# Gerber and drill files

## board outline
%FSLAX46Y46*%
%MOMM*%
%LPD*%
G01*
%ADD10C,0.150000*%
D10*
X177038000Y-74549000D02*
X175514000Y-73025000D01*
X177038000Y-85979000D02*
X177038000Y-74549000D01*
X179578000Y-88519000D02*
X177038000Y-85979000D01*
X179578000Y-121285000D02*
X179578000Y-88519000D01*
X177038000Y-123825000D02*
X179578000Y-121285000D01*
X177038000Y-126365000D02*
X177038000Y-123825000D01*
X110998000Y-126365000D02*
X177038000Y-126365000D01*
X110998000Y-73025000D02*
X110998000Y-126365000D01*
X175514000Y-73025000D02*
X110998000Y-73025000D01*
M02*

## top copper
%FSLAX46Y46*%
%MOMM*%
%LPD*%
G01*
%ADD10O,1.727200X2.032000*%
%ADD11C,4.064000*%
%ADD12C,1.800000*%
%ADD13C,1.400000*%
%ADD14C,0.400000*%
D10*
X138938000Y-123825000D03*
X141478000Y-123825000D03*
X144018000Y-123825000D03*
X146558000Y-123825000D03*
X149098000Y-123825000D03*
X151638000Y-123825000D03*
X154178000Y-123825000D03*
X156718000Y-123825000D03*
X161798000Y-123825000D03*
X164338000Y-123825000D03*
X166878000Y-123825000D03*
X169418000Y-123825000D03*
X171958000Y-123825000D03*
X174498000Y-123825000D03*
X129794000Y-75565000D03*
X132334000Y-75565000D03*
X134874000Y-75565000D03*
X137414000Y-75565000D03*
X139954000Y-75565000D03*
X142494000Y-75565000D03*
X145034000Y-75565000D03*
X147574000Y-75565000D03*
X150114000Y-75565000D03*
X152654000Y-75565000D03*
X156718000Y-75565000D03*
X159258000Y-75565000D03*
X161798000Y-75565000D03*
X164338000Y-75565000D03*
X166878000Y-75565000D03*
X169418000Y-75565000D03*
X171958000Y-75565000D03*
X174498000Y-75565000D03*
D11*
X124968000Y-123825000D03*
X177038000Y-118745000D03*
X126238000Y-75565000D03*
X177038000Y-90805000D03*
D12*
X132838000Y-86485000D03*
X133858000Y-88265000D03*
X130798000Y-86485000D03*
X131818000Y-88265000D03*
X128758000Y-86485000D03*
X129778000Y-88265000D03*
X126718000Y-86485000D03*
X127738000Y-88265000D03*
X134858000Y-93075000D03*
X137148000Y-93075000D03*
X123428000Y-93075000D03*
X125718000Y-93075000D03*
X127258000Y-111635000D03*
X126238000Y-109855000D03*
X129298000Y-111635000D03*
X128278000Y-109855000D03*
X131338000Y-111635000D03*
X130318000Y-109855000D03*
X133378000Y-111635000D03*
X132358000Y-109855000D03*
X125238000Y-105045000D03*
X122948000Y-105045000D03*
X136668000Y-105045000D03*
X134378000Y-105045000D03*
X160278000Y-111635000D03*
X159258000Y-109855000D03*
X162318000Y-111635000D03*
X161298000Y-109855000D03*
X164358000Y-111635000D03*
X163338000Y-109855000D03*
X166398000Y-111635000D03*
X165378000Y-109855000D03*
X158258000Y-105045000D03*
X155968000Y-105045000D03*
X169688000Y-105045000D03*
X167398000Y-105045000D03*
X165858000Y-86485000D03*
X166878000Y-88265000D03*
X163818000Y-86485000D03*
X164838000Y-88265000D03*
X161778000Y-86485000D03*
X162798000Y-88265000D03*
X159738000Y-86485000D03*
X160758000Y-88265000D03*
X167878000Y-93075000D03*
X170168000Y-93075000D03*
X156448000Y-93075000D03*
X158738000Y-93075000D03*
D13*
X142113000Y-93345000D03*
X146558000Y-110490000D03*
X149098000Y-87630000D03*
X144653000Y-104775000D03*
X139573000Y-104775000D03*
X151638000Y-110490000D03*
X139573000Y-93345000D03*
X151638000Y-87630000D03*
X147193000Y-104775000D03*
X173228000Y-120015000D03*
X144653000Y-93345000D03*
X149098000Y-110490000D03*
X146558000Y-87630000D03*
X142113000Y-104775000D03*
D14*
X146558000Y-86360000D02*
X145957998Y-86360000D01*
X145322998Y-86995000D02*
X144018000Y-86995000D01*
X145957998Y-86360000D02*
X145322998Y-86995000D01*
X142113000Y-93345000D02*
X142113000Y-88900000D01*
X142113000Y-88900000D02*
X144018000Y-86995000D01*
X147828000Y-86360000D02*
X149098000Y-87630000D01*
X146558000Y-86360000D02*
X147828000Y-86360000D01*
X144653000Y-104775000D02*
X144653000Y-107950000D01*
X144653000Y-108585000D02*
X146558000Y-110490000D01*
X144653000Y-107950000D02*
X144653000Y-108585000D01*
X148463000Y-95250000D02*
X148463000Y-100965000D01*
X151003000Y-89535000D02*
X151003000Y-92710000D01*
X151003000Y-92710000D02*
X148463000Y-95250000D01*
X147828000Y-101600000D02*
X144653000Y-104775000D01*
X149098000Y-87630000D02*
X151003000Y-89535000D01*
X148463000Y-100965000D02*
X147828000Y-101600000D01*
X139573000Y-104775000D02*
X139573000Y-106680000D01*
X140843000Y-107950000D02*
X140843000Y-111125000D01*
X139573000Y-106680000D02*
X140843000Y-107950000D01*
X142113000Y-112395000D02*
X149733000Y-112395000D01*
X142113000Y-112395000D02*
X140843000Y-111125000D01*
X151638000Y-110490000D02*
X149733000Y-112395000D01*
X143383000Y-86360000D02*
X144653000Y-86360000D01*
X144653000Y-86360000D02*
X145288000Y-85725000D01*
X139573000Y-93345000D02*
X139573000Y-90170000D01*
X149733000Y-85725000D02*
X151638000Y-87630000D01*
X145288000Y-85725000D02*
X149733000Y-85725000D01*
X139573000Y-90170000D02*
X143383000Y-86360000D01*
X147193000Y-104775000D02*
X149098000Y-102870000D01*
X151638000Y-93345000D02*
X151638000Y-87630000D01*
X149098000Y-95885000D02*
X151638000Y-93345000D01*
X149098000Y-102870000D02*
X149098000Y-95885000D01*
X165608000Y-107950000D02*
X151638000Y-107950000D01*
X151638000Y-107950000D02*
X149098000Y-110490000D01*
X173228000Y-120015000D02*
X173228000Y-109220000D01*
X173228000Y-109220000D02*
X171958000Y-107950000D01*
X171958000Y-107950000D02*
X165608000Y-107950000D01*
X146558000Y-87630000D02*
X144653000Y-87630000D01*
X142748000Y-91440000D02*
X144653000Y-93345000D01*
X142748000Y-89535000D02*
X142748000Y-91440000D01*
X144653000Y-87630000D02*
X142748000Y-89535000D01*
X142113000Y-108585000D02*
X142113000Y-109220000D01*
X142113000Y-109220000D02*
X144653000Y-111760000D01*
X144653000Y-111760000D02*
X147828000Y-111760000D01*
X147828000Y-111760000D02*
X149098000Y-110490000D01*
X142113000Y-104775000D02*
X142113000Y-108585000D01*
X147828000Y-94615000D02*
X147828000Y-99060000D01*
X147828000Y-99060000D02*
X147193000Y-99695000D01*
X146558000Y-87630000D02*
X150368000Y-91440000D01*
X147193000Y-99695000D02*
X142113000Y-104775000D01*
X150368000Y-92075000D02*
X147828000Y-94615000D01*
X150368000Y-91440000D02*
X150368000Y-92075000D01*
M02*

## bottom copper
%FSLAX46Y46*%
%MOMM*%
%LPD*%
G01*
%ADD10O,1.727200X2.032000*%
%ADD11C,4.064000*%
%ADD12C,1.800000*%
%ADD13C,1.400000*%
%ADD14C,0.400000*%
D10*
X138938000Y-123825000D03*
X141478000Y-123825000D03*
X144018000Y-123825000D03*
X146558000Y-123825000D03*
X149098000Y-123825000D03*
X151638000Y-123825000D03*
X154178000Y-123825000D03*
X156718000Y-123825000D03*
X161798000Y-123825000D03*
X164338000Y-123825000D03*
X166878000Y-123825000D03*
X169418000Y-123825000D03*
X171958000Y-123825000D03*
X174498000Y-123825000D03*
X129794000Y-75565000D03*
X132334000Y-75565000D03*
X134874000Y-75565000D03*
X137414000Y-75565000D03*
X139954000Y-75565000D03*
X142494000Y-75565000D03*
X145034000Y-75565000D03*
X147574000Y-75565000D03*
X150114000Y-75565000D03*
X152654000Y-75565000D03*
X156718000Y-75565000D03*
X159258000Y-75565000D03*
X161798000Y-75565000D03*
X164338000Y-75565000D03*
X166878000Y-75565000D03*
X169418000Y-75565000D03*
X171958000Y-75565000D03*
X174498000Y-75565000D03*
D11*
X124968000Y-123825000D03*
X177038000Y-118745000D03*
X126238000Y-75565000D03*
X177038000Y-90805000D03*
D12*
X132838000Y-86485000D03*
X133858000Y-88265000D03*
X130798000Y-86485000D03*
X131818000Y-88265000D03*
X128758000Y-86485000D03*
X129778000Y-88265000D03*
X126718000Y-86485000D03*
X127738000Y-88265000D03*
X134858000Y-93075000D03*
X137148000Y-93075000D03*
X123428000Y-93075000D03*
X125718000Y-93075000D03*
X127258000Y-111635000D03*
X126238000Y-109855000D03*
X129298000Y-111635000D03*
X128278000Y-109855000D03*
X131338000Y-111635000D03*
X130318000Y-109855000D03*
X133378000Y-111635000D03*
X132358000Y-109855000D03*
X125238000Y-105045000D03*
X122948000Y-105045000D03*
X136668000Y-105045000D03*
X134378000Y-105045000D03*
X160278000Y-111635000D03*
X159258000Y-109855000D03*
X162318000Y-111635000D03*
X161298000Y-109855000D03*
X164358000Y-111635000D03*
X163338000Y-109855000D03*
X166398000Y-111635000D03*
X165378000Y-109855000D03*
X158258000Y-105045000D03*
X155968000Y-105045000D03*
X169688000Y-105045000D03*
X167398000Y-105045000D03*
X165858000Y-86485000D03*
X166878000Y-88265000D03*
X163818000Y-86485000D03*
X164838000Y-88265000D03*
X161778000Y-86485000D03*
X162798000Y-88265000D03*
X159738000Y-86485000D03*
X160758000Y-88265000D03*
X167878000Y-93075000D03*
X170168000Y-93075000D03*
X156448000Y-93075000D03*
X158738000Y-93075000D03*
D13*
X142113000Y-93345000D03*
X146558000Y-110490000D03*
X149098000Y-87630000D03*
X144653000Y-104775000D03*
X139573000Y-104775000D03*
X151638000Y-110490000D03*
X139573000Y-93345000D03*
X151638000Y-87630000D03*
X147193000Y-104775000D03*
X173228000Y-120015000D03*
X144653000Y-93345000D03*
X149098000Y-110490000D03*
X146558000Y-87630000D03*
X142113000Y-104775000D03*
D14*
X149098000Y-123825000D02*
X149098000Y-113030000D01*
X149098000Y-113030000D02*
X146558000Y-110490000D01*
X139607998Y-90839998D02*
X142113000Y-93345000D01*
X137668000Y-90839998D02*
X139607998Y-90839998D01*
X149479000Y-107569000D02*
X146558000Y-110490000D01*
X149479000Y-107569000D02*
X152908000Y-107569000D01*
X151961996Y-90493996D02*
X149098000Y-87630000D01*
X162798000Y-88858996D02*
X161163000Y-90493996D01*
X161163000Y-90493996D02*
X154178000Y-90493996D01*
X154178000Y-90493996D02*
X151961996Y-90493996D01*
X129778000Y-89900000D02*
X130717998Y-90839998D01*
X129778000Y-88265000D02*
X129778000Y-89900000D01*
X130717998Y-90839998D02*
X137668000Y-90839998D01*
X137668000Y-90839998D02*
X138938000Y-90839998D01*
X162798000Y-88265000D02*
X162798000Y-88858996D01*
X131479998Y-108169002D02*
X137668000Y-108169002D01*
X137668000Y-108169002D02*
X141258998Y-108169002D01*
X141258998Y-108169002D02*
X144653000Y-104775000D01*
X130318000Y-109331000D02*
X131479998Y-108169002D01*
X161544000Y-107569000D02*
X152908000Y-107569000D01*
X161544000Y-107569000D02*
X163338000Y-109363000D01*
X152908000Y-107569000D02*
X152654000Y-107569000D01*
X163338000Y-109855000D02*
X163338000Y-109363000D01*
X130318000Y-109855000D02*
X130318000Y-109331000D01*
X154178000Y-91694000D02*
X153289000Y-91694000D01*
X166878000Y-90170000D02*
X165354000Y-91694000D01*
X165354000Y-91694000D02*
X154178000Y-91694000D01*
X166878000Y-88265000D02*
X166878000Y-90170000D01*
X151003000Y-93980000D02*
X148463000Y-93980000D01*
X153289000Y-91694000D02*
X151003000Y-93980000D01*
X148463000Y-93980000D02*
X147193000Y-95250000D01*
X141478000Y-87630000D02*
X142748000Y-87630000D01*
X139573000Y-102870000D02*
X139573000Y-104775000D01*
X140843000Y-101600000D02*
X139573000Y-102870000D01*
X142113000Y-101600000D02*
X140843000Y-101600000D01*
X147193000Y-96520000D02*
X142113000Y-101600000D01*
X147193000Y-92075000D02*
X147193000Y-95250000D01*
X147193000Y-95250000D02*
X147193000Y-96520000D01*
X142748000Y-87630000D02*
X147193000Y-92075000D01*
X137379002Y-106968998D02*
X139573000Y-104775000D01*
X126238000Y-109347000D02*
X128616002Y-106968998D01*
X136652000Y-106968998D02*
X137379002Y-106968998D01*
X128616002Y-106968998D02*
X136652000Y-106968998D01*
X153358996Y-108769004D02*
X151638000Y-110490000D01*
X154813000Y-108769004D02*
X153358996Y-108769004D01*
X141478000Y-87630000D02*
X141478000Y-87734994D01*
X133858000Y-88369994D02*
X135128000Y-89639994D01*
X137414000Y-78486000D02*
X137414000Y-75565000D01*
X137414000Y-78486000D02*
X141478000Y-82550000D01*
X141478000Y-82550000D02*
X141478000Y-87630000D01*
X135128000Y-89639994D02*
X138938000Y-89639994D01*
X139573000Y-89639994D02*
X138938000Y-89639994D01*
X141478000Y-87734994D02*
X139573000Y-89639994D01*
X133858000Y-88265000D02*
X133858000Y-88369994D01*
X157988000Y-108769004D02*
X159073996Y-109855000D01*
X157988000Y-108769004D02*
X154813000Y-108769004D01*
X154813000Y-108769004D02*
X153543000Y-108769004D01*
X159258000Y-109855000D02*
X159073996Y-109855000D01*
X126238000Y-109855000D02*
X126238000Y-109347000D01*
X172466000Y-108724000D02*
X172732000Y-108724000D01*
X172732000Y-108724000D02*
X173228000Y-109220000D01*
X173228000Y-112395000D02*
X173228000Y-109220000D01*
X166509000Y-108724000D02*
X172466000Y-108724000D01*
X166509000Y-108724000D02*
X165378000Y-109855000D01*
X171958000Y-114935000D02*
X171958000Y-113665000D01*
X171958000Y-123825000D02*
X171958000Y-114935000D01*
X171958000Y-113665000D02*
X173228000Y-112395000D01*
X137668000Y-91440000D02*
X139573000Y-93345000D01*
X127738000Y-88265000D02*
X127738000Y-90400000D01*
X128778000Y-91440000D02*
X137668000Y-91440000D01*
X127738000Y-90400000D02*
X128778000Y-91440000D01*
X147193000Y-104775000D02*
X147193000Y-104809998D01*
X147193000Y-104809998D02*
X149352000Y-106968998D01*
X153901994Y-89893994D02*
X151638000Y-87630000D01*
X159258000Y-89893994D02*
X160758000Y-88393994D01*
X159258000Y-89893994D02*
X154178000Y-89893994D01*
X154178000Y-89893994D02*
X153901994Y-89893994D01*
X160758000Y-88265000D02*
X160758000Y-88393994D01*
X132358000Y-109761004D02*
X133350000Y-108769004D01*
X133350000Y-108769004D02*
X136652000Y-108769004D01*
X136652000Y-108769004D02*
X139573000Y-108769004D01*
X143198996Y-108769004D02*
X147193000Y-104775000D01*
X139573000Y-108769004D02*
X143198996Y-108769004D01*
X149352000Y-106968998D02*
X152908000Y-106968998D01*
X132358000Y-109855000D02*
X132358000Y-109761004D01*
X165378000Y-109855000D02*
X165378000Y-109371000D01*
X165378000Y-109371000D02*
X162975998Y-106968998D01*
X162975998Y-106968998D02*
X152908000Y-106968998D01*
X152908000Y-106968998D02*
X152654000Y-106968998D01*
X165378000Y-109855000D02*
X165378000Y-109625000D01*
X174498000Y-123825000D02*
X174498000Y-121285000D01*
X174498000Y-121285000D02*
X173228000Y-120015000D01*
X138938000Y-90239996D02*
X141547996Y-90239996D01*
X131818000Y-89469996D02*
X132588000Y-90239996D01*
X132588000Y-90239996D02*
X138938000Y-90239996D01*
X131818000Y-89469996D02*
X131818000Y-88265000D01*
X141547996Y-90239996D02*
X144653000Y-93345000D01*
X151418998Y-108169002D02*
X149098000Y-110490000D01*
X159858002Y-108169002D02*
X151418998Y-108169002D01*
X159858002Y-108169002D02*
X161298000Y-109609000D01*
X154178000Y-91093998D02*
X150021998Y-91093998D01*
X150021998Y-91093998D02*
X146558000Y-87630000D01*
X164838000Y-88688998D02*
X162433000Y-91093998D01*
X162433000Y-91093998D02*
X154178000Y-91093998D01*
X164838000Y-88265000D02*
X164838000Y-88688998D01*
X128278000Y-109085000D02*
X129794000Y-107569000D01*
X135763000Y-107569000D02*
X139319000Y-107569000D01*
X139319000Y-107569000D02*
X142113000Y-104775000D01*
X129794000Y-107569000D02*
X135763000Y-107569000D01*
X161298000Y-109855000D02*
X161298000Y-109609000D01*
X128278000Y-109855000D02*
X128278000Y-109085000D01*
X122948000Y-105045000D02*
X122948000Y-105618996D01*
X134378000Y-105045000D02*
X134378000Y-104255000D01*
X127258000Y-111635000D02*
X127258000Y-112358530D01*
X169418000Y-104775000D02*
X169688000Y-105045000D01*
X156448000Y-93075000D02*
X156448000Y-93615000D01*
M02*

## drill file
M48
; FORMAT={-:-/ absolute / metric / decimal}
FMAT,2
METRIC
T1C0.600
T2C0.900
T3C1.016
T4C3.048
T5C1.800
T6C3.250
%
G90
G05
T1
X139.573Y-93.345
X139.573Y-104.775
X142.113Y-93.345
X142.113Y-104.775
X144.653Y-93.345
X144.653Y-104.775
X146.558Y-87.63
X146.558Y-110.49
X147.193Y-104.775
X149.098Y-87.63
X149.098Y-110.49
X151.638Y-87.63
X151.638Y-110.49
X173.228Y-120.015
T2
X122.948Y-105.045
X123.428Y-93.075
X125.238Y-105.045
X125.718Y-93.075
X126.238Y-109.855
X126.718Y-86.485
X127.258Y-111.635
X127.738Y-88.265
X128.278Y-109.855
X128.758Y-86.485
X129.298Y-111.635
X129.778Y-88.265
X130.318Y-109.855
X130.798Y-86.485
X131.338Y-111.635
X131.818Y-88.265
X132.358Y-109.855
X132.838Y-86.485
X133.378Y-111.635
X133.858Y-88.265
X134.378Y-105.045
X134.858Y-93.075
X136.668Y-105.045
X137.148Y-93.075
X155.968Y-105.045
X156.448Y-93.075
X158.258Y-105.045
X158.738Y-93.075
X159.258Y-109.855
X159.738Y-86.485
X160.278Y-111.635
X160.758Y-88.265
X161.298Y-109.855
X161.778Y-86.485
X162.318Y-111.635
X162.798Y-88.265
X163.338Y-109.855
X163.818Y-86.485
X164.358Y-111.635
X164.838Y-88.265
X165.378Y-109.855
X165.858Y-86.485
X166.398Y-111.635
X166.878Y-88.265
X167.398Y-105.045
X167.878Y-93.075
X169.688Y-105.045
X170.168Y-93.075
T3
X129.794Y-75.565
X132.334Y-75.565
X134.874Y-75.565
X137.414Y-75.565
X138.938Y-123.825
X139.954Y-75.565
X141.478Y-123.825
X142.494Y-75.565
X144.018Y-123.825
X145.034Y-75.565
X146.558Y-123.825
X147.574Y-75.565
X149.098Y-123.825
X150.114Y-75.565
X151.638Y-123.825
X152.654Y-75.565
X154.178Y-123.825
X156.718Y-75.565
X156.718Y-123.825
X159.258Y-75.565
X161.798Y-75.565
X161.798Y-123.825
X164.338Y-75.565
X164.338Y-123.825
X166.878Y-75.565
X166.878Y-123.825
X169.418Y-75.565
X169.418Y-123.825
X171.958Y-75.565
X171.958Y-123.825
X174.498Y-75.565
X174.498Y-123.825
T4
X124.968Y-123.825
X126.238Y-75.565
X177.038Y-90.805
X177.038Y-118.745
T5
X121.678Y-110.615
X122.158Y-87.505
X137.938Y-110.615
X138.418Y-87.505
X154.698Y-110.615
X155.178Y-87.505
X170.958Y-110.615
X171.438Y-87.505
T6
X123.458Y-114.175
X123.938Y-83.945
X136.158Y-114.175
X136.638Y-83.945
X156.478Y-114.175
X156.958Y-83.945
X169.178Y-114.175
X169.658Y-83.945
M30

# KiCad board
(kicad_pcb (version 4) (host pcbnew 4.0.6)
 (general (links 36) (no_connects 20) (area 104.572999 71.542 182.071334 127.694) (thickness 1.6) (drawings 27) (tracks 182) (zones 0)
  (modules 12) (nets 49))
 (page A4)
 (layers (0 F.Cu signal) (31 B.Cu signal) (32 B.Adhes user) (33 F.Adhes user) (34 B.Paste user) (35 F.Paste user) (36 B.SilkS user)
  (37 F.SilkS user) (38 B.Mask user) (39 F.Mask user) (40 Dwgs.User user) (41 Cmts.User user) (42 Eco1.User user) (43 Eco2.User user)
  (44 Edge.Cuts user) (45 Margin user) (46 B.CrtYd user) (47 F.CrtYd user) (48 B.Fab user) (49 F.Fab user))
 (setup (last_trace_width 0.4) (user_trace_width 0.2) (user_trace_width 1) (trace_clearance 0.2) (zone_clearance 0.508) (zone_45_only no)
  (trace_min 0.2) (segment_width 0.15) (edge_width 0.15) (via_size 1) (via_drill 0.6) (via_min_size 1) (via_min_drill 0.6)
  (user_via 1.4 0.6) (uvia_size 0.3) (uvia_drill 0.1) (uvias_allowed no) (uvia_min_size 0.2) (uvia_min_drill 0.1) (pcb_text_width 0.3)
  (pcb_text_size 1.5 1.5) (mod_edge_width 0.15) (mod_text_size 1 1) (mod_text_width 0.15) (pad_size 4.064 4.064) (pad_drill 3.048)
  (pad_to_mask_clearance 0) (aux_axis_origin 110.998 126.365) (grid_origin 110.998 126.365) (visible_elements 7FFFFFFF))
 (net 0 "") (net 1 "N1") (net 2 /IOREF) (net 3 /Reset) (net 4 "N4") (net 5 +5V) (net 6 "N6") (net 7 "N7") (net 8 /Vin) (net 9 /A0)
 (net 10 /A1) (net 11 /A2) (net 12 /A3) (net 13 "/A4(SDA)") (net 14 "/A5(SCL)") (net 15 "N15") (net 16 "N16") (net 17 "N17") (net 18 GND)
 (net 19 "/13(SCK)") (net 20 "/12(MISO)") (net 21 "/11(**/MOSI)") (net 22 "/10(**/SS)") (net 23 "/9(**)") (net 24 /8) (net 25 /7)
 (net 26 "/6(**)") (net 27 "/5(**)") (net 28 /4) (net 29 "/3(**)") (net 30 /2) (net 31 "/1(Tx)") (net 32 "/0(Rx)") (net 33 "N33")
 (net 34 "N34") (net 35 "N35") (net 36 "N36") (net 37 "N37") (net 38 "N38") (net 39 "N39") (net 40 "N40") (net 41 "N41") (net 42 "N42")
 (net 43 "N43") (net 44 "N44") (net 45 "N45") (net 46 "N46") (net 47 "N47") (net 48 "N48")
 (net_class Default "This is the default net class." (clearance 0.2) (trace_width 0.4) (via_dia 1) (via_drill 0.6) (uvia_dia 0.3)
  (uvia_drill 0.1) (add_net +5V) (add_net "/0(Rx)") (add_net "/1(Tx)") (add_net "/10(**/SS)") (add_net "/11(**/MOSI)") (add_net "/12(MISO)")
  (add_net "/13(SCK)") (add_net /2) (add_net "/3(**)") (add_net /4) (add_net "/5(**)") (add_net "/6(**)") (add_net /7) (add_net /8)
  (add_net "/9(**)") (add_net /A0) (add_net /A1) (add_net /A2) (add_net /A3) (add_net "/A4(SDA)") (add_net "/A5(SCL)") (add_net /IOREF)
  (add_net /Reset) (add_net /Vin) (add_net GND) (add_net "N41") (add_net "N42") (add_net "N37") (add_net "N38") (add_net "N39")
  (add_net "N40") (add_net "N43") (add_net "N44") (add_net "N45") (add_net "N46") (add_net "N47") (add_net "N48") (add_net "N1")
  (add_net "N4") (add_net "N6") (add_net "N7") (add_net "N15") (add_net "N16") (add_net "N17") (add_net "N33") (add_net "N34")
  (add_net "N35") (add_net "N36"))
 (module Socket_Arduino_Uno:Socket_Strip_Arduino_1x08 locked (layer F.Cu) (at 138.938 123.825)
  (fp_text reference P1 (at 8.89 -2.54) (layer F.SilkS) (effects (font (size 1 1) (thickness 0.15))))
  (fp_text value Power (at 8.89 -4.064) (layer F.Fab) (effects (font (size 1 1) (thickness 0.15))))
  (pad 1 thru_hole oval (at 0 0) (size 1.7272 2.032) (drill 1.016) (layers *.Cu *.Mask F.SilkS) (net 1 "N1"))
  (pad 2 thru_hole oval (at 2.54 0) (size 1.7272 2.032) (drill 1.016) (layers *.Cu *.Mask F.SilkS) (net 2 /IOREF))
  (pad 3 thru_hole oval (at 5.08 0) (size 1.7272 2.032) (drill 1.016) (layers *.Cu *.Mask F.SilkS) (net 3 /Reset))
  (pad 4 thru_hole oval (at 7.62 0) (size 1.7272 2.032) (drill 1.016) (layers *.Cu *.Mask F.SilkS) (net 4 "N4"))
  (pad 5 thru_hole oval (at 10.16 0) (size 1.7272 2.032) (drill 1.016) (layers *.Cu *.Mask F.SilkS) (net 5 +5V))
  (pad 6 thru_hole oval (at 12.7 0) (size 1.7272 2.032) (drill 1.016) (layers *.Cu *.Mask F.SilkS) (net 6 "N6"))
  (pad 7 thru_hole oval (at 15.24 0) (size 1.7272 2.032) (drill 1.016) (layers *.Cu *.Mask F.SilkS) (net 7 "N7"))
  (pad 8 thru_hole oval (at 17.78 0) (size 1.7272 2.032) (drill 1.016) (layers *.Cu *.Mask F.SilkS) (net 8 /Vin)))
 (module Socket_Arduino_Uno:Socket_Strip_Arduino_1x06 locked (layer F.Cu) (at 161.798 123.825)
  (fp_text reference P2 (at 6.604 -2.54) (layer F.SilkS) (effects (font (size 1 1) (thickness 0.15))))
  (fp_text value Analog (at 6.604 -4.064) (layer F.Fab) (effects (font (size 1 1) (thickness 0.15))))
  (pad 1 thru_hole oval (at 0 0) (size 1.7272 2.032) (drill 1.016) (layers *.Cu *.Mask F.SilkS) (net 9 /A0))
  (pad 2 thru_hole oval (at 2.54 0) (size 1.7272 2.032) (drill 1.016) (layers *.Cu *.Mask F.SilkS) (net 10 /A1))
  (pad 3 thru_hole oval (at 5.08 0) (size 1.7272 2.032) (drill 1.016) (layers *.Cu *.Mask F.SilkS) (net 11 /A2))
  (pad 4 thru_hole oval (at 7.62 0) (size 1.7272 2.032) (drill 1.016) (layers *.Cu *.Mask F.SilkS) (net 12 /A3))
  (pad 5 thru_hole oval (at 10.16 0) (size 1.7272 2.032) (drill 1.016) (layers *.Cu *.Mask F.SilkS) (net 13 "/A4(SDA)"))
  (pad 6 thru_hole oval (at 12.7 0) (size 1.7272 2.032) (drill 1.016) (layers *.Cu *.Mask F.SilkS) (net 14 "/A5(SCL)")))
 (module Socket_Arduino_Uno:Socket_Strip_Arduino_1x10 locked (layer F.Cu) (at 129.794 75.565)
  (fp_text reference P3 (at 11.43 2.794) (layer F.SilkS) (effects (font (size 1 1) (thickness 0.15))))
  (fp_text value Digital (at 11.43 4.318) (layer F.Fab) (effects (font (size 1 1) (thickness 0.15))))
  (pad 1 thru_hole oval (at 0 0) (size 1.7272 2.032) (drill 1.016) (layers *.Cu *.Mask F.SilkS) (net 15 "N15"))
  (pad 2 thru_hole oval (at 2.54 0) (size 1.7272 2.032) (drill 1.016) (layers *.Cu *.Mask F.SilkS) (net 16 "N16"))
  (pad 3 thru_hole oval (at 5.08 0) (size 1.7272 2.032) (drill 1.016) (layers *.Cu *.Mask F.SilkS) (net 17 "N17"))
  (pad 4 thru_hole oval (at 7.62 0) (size 1.7272 2.032) (drill 1.016) (layers *.Cu *.Mask F.SilkS) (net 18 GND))
  (pad 5 thru_hole oval (at 10.16 0) (size 1.7272 2.032) (drill 1.016) (layers *.Cu *.Mask F.SilkS) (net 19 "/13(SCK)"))
  (pad 6 thru_hole oval (at 12.7 0) (size 1.7272 2.032) (drill 1.016) (layers *.Cu *.Mask F.SilkS) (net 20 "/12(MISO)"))
  (pad 7 thru_hole oval (at 15.24 0) (size 1.7272 2.032) (drill 1.016) (layers *.Cu *.Mask F.SilkS) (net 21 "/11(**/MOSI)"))
  (pad 8 thru_hole oval (at 17.78 0) (size 1.7272 2.032) (drill 1.016) (layers *.Cu *.Mask F.SilkS) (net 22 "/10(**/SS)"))
  (pad 9 thru_hole oval (at 20.32 0) (size 1.7272 2.032) (drill 1.016) (layers *.Cu *.Mask F.SilkS) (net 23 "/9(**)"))
  (pad 10 thru_hole oval (at 22.86 0) (size 1.7272 2.032) (drill 1.016) (layers *.Cu *.Mask F.SilkS) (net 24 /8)))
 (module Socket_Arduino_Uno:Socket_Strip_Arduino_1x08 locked (layer F.Cu) (at 156.718 75.565)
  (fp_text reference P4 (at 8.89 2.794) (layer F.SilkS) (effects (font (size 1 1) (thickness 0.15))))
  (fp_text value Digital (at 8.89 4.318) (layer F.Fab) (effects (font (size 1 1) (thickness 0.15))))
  (pad 1 thru_hole oval (at 0 0) (size 1.7272 2.032) (drill 1.016) (layers *.Cu *.Mask F.SilkS) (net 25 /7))
  (pad 2 thru_hole oval (at 2.54 0) (size 1.7272 2.032) (drill 1.016) (layers *.Cu *.Mask F.SilkS) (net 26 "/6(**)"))
  (pad 3 thru_hole oval (at 5.08 0) (size 1.7272 2.032) (drill 1.016) (layers *.Cu *.Mask F.SilkS) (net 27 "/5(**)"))
  (pad 4 thru_hole oval (at 7.62 0) (size 1.7272 2.032) (drill 1.016) (layers *.Cu *.Mask F.SilkS) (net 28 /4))
  (pad 5 thru_hole oval (at 10.16 0) (size 1.7272 2.032) (drill 1.016) (layers *.Cu *.Mask F.SilkS) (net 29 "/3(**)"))
  (pad 6 thru_hole oval (at 12.7 0) (size 1.7272 2.032) (drill 1.016) (layers *.Cu *.Mask F.SilkS) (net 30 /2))
  (pad 7 thru_hole oval (at 15.24 0) (size 1.7272 2.032) (drill 1.016) (layers *.Cu *.Mask F.SilkS) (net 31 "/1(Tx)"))
  (pad 8 thru_hole oval (at 17.78 0) (size 1.7272 2.032) (drill 1.016) (layers *.Cu *.Mask F.SilkS) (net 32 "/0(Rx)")))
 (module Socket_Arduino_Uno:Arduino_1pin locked (layer F.Cu) (at 124.968 123.825)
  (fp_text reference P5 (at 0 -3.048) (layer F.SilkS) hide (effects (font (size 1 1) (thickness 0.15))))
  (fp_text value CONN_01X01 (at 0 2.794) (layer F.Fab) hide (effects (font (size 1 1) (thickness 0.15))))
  (pad 1 thru_hole circle (at 0 0) (size 4.064 4.064) (drill 3.048) (layers *.Cu *.Mask F.SilkS) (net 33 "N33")))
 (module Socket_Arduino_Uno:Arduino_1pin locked (layer F.Cu) (at 177.038 118.745)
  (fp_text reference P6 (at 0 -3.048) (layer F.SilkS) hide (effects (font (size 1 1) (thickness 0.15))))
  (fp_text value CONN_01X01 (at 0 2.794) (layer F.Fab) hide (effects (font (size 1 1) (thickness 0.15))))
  (pad 1 thru_hole circle (at 0 0) (size 4.064 4.064) (drill 3.048) (layers *.Cu *.Mask F.SilkS) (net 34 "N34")))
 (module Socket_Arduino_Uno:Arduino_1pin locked (layer F.Cu) (at 126.238 75.565)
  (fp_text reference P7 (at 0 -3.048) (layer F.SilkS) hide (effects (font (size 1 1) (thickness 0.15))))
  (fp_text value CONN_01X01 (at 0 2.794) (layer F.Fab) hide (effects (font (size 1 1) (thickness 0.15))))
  (pad 1 thru_hole circle (at 0 0) (size 4.064 4.064) (drill 3.048) (layers *.Cu *.Mask F.SilkS) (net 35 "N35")))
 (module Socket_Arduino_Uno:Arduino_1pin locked (layer F.Cu) (at 177.038 90.805)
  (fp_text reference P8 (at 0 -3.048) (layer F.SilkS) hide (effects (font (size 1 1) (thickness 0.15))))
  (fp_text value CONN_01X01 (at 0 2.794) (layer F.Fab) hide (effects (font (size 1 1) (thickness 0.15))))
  (pad 1 thru_hole circle (at 0 0) (size 4.064 4.064) (drill 3.048) (layers *.Cu *.Mask F.SilkS) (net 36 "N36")))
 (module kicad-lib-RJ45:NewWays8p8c (layer F.Cu) (at 133.858 88.265 180)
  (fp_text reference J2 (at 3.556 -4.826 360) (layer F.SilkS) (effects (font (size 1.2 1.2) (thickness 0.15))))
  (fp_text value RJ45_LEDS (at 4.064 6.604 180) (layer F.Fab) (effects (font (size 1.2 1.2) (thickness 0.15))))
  (pad 2 thru_hole circle (at 1.02 1.78 180) (size 1.8 1.8) (drill 0.9) (layers *.Cu *.Mask) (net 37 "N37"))
  (pad 1 thru_hole circle (at 0 0 180) (size 1.8 1.8) (drill 0.9) (layers *.Cu *.Mask) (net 18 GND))
  (pad 4 thru_hole circle (at 3.06 1.78 180) (size 1.8 1.8) (drill 0.9) (layers *.Cu *.Mask) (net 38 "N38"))
  (pad 3 thru_hole circle (at 2.04 0 180) (size 1.8 1.8) (drill 0.9) (layers *.Cu *.Mask) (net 14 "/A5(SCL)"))
  (pad 6 thru_hole circle (at 5.1 1.78 180) (size 1.8 1.8) (drill 0.9) (layers *.Cu *.Mask) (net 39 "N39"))
  (pad 5 thru_hole circle (at 4.08 0 180) (size 1.8 1.8) (drill 0.9) (layers *.Cu *.Mask) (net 5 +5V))
  (pad 8 thru_hole circle (at 7.14 1.78 180) (size 1.8 1.8) (drill 0.9) (layers *.Cu *.Mask) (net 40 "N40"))
  (pad 7 thru_hole circle (at 6.12 0 180) (size 1.8 1.8) (drill 0.9) (layers *.Cu *.Mask) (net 13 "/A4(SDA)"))
  (pad 10 thru_hole circle (at -1 -4.81 180) (size 1.8 1.8) (drill 0.9) (layers *.Cu *.Mask) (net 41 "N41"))
  (pad 9 thru_hole circle (at -3.29 -4.81 180) (size 1.8 1.8) (drill 0.9) (layers *.Cu *.Mask) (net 20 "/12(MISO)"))
  (pad 12 thru_hole circle (at 10.43 -4.81 180) (size 1.8 1.8) (drill 0.9) (layers *.Cu *.Mask) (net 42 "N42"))
  (pad 11 thru_hole circle (at 8.14 -4.81 180) (size 1.8 1.8) (drill 0.9) (layers *.Cu *.Mask) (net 19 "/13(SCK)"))
  (pad "" np_thru_hole circle (at -2.78 4.32 180) (size 3.25 3.25) (drill 3.25) (layers *.Cu *.Mask))
  (pad "" np_thru_hole circle (at 9.92 4.32 180) (size 3.25 3.25) (drill 3.25) (layers *.Cu *.Mask))
  (pad "" np_thru_hole circle (at -4.56 0.76 180) (size 1.8 1.8) (drill 1.8) (layers *.Cu *.Mask))
  (pad "" np_thru_hole circle (at 11.7 0.76 180) (size 1.8 1.8) (drill 1.8) (layers *.Cu *.Mask)))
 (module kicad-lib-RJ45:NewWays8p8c (layer F.Cu) (at 126.238 109.855)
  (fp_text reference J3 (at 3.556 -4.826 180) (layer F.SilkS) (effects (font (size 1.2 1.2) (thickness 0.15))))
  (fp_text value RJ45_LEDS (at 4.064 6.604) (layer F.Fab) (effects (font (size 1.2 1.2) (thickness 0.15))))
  (pad 2 thru_hole circle (at 1.02 1.78) (size 1.8 1.8) (drill 0.9) (layers *.Cu *.Mask) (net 37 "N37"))
  (pad 1 thru_hole circle (at 0 0) (size 1.8 1.8) (drill 0.9) (layers *.Cu *.Mask) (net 18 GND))
  (pad 4 thru_hole circle (at 3.06 1.78) (size 1.8 1.8) (drill 0.9) (layers *.Cu *.Mask) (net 38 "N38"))
  (pad 3 thru_hole circle (at 2.04 0) (size 1.8 1.8) (drill 0.9) (layers *.Cu *.Mask) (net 14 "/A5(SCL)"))
  (pad 6 thru_hole circle (at 5.1 1.78) (size 1.8 1.8) (drill 0.9) (layers *.Cu *.Mask) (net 39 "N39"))
  (pad 5 thru_hole circle (at 4.08 0) (size 1.8 1.8) (drill 0.9) (layers *.Cu *.Mask) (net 5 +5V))
  (pad 8 thru_hole circle (at 7.14 1.78) (size 1.8 1.8) (drill 0.9) (layers *.Cu *.Mask) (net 40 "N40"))
  (pad 7 thru_hole circle (at 6.12 0) (size 1.8 1.8) (drill 0.9) (layers *.Cu *.Mask) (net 13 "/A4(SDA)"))
  (pad 10 thru_hole circle (at -1 -4.81) (size 1.8 1.8) (drill 0.9) (layers *.Cu *.Mask) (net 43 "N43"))
  (pad 9 thru_hole circle (at -3.29 -4.81) (size 1.8 1.8) (drill 0.9) (layers *.Cu *.Mask) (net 22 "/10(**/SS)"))
  (pad 12 thru_hole circle (at 10.43 -4.81) (size 1.8 1.8) (drill 0.9) (layers *.Cu *.Mask) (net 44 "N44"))
  (pad 11 thru_hole circle (at 8.14 -4.81) (size 1.8 1.8) (drill 0.9) (layers *.Cu *.Mask) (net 21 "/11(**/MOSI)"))
  (pad "" np_thru_hole circle (at -2.78 4.32) (size 3.25 3.25) (drill 3.25) (layers *.Cu *.Mask))
  (pad "" np_thru_hole circle (at 9.92 4.32) (size 3.25 3.25) (drill 3.25) (layers *.Cu *.Mask))
  (pad "" np_thru_hole circle (at -4.56 0.76) (size 1.8 1.8) (drill 1.8) (layers *.Cu *.Mask))
  (pad "" np_thru_hole circle (at 11.7 0.76) (size 1.8 1.8) (drill 1.8) (layers *.Cu *.Mask)))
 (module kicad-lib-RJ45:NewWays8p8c (layer F.Cu) (at 159.258 109.855)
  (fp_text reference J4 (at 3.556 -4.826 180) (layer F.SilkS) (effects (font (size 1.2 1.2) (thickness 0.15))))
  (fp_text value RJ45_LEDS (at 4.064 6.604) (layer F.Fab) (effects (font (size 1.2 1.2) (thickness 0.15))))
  (pad 2 thru_hole circle (at 1.02 1.78) (size 1.8 1.8) (drill 0.9) (layers *.Cu *.Mask) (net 37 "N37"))
  (pad 1 thru_hole circle (at 0 0) (size 1.8 1.8) (drill 0.9) (layers *.Cu *.Mask) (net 18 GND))
  (pad 4 thru_hole circle (at 3.06 1.78) (size 1.8 1.8) (drill 0.9) (layers *.Cu *.Mask) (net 38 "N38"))
  (pad 3 thru_hole circle (at 2.04 0) (size 1.8 1.8) (drill 0.9) (layers *.Cu *.Mask) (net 14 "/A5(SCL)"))
  (pad 6 thru_hole circle (at 5.1 1.78) (size 1.8 1.8) (drill 0.9) (layers *.Cu *.Mask) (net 39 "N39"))
  (pad 5 thru_hole circle (at 4.08 0) (size 1.8 1.8) (drill 0.9) (layers *.Cu *.Mask) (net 5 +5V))
  (pad 8 thru_hole circle (at 7.14 1.78) (size 1.8 1.8) (drill 0.9) (layers *.Cu *.Mask) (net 40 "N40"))
  (pad 7 thru_hole circle (at 6.12 0) (size 1.8 1.8) (drill 0.9) (layers *.Cu *.Mask) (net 13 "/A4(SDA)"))
  (pad 10 thru_hole circle (at -1 -4.81) (size 1.8 1.8) (drill 0.9) (layers *.Cu *.Mask) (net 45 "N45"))
  (pad 9 thru_hole circle (at -3.29 -4.81) (size 1.8 1.8) (drill 0.9) (layers *.Cu *.Mask) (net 24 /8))
  (pad 12 thru_hole circle (at 10.43 -4.81) (size 1.8 1.8) (drill 0.9) (layers *.Cu *.Mask) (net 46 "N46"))
  (pad 11 thru_hole circle (at 8.14 -4.81) (size 1.8 1.8) (drill 0.9) (layers *.Cu *.Mask) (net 23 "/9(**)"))
  (pad "" np_thru_hole circle (at -2.78 4.32) (size 3.25 3.25) (drill 3.25) (layers *.Cu *.Mask))
  (pad "" np_thru_hole circle (at 9.92 4.32) (size 3.25 3.25) (drill 3.25) (layers *.Cu *.Mask))
  (pad "" np_thru_hole circle (at -4.56 0.76) (size 1.8 1.8) (drill 1.8) (layers *.Cu *.Mask))
  (pad "" np_thru_hole circle (at 11.7 0.76) (size 1.8 1.8) (drill 1.8) (layers *.Cu *.Mask)))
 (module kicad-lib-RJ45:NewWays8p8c (layer F.Cu) (at 166.878 88.265 180)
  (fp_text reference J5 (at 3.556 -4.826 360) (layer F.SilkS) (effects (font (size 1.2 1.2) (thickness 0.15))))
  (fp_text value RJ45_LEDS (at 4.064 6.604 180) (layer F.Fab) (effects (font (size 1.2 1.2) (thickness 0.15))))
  (pad 2 thru_hole circle (at 1.02 1.78 180) (size 1.8 1.8) (drill 0.9) (layers *.Cu *.Mask) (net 37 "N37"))
  (pad 1 thru_hole circle (at 0 0 180) (size 1.8 1.8) (drill 0.9) (layers *.Cu *.Mask) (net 18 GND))
  (pad 4 thru_hole circle (at 3.06 1.78 180) (size 1.8 1.8) (drill 0.9) (layers *.Cu *.Mask) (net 38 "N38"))
  (pad 3 thru_hole circle (at 2.04 0 180) (size 1.8 1.8) (drill 0.9) (layers *.Cu *.Mask) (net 14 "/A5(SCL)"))
  (pad 6 thru_hole circle (at 5.1 1.78 180) (size 1.8 1.8) (drill 0.9) (layers *.Cu *.Mask) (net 39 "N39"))
  (pad 5 thru_hole circle (at 4.08 0 180) (size 1.8 1.8) (drill 0.9) (layers *.Cu *.Mask) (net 5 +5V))
  (pad 8 thru_hole circle (at 7.14 1.78 180) (size 1.8 1.8) (drill 0.9) (layers *.Cu *.Mask) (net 40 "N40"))
  (pad 7 thru_hole circle (at 6.12 0 180) (size 1.8 1.8) (drill 0.9) (layers *.Cu *.Mask) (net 13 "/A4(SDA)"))
  (pad 10 thru_hole circle (at -1 -4.81 180) (size 1.8 1.8) (drill 0.9) (layers *.Cu *.Mask) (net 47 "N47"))
  (pad 9 thru_hole circle (at -3.29 -4.81 180) (size 1.8 1.8) (drill 0.9) (layers *.Cu *.Mask) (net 26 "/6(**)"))
  (pad 12 thru_hole circle (at 10.43 -4.81 180) (size 1.8 1.8) (drill 0.9) (layers *.Cu *.Mask) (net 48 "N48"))
  (pad 11 thru_hole circle (at 8.14 -4.81 180) (size 1.8 1.8) (drill 0.9) (layers *.Cu *.Mask) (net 25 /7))
  (pad "" np_thru_hole circle (at -2.78 4.32 180) (size 3.25 3.25) (drill 3.25) (layers *.Cu *.Mask))
  (pad "" np_thru_hole circle (at 9.92 4.32 180) (size 3.25 3.25) (drill 3.25) (layers *.Cu *.Mask))
  (pad "" np_thru_hole circle (at -4.56 0.76 180) (size 1.8 1.8) (drill 1.8) (layers *.Cu *.Mask))
  (pad "" np_thru_hole circle (at 11.7 0.76 180) (size 1.8 1.8) (drill 1.8) (layers *.Cu *.Mask)))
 (gr_line (start 177.038 74.549) (end 175.514 73.025) (angle 90) (layer Edge.Cuts) (width 0.15))
 (gr_line (start 177.038 85.979) (end 177.038 74.549) (angle 90) (layer Edge.Cuts) (width 0.15))
 (gr_line (start 179.578 88.519) (end 177.038 85.979) (angle 90) (layer Edge.Cuts) (width 0.15))
 (gr_line (start 179.578 121.285) (end 179.578 88.519) (angle 90) (layer Edge.Cuts) (width 0.15))
 (gr_line (start 177.038 123.825) (end 179.578 121.285) (angle 90) (layer Edge.Cuts) (width 0.15))
 (gr_line (start 177.038 126.365) (end 177.038 123.825) (angle 90) (layer Edge.Cuts) (width 0.15))
 (gr_line (start 110.998 126.365) (end 177.038 126.365) (angle 90) (layer Edge.Cuts) (width 0.15))
 (gr_line (start 110.998 73.025) (end 110.998 126.365) (angle 90) (layer Edge.Cuts) (width 0.15))
 (gr_line (start 175.514 73.025) (end 110.998 73.025) (angle 90) (layer Edge.Cuts) (width 0.15))
 (segment (start 149.098 123.825) (end 149.098 113.03) (width 0.4) (layer B.Cu) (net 5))
 (segment (start 149.098 113.03) (end 146.558 110.49) (width 0.4) (layer B.Cu) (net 5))
 (segment (start 146.558 86.36) (end 145.957998 86.36) (width 0.4) (layer F.Cu) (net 5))
 (segment (start 145.322998 86.995) (end 144.018 86.995) (width 0.4) (layer F.Cu) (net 5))
 (segment (start 145.957998 86.36) (end 145.322998 86.995) (width 0.4) (layer F.Cu) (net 5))
 (segment (start 142.113 93.345) (end 142.113 88.9) (width 0.4) (layer F.Cu) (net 5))
 (segment (start 142.113 88.9) (end 144.018 86.995) (width 0.4) (layer F.Cu) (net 5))
 (segment (start 139.607998 90.839998) (end 142.113 93.345) (width 0.4) (layer B.Cu) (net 5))
 (via (at 142.113 93.345) (size 1.4) (drill 0.6) (layers F.Cu B.Cu) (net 5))
 (segment (start 137.668 90.839998) (end 139.607998 90.839998) (width 0.4) (layer B.Cu) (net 5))
 (segment (start 147.828 86.36) (end 149.098 87.63) (width 0.4) (layer F.Cu) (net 5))
 (segment (start 146.558 86.36) (end 147.828 86.36) (width 0.4) (layer F.Cu) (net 5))
 (segment (start 144.653 104.775) (end 144.653 107.95) (width 0.4) (layer F.Cu) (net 5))
 (segment (start 144.653 108.585) (end 146.558 110.49) (width 0.4) (layer F.Cu) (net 5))
 (segment (start 144.653 107.95) (end 144.653 108.585) (width 0.4) (layer F.Cu) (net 5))
 (segment (start 149.479 107.569) (end 146.558 110.49) (width 0.4) (layer B.Cu) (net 5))
 (segment (start 149.479 107.569) (end 152.908 107.569) (width 0.4) (layer B.Cu) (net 5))
 (via (at 146.558 110.49) (size 1.4) (drill 0.6) (layers F.Cu B.Cu) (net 5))
 (segment (start 148.463 95.25) (end 148.463 100.965) (width 0.4) (layer F.Cu) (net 5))
 (segment (start 151.003 89.535) (end 151.003 92.71) (width 0.4) (layer F.Cu) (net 5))
 (segment (start 151.003 92.71) (end 148.463 95.25) (width 0.4) (layer F.Cu) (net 5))
 (segment (start 147.828 101.6) (end 144.653 104.775) (width 0.4) (layer F.Cu) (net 5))
 (segment (start 149.098 87.63) (end 151.003 89.535) (width 0.4) (layer F.Cu) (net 5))
 (segment (start 148.463 100.965) (end 147.828 101.6) (width 0.4) (layer F.Cu) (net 5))
 (segment (start 151.961996 90.493996) (end 149.098 87.63) (width 0.4) (layer B.Cu) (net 5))
 (via (at 149.098 87.63) (size 1.4) (drill 0.6) (layers F.Cu B.Cu) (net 5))
 (segment (start 162.798 88.858996) (end 161.163 90.493996) (width 0.4) (layer B.Cu) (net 5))
 (segment (start 161.163 90.493996) (end 154.178 90.493996) (width 0.4) (layer B.Cu) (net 5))
 (segment (start 154.178 90.493996) (end 151.961996 90.493996) (width 0.4) (layer B.Cu) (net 5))
 (segment (start 129.778 89.9) (end 130.717998 90.839998) (width 0.4) (layer B.Cu) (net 5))
 (segment (start 129.778 88.265) (end 129.778 89.9) (width 0.4) (layer B.Cu) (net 5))
 (segment (start 130.717998 90.839998) (end 137.668 90.839998) (width 0.4) (layer B.Cu) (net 5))
 (segment (start 137.668 90.839998) (end 138.938 90.839998) (width 0.4) (layer B.Cu) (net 5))
 (segment (start 162.798 88.265) (end 162.798 88.858996) (width 0.4) (layer B.Cu) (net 5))
 (segment (start 131.479998 108.169002) (end 137.668 108.169002) (width 0.4) (layer B.Cu) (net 5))
 (segment (start 137.668 108.169002) (end 141.258998 108.169002) (width 0.4) (layer B.Cu) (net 5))
 (via (at 144.653 104.775) (size 1.4) (drill 0.6) (layers F.Cu B.Cu) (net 5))
 (segment (start 141.258998 108.169002) (end 144.653 104.775) (width 0.4) (layer B.Cu) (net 5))
 (segment (start 130.318 109.331) (end 131.479998 108.169002) (width 0.4) (layer B.Cu) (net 5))
 (segment (start 161.544 107.569) (end 152.908 107.569) (width 0.4) (layer B.Cu) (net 5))
 (segment (start 161.544 107.569) (end 163.338 109.363) (width 0.4) (layer B.Cu) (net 5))
 (segment (start 152.908 107.569) (end 152.654 107.569) (width 0.4) (layer B.Cu) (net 5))
 (segment (start 163.338 109.855) (end 163.338 109.363) (width 0.4) (layer B.Cu) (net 5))
 (segment (start 130.318 109.855) (end 130.318 109.331) (width 0.4) (layer B.Cu) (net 5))
 (segment (start 154.178 91.694) (end 153.289 91.694) (width 0.4) (layer B.Cu) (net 18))
 (segment (start 166.878 90.17) (end 165.354 91.694) (width 0.4) (layer B.Cu) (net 18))
 (segment (start 165.354 91.694) (end 154.178 91.694) (width 0.4) (layer B.Cu) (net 18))
 (segment (start 166.878 88.265) (end 166.878 90.17) (width 0.4) (layer B.Cu) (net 18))
 (segment (start 151.003 93.98) (end 148.463 93.98) (width 0.4) (layer B.Cu) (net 18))
 (segment (start 153.289 91.694) (end 151.003 93.98) (width 0.4) (layer B.Cu) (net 18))
 (segment (start 148.463 93.98) (end 147.193 95.25) (width 0.4) (layer B.Cu) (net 18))
 (segment (start 141.478 87.63) (end 142.748 87.63) (width 0.4) (layer B.Cu) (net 18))
 (segment (start 139.573 102.87) (end 139.573 104.775) (width 0.4) (layer B.Cu) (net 18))
 (segment (start 140.843 101.6) (end 139.573 102.87) (width 0.4) (layer B.Cu) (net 18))
 (segment (start 142.113 101.6) (end 140.843 101.6) (width 0.4) (layer B.Cu) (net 18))
 (segment (start 147.193 96.52) (end 142.113 101.6) (width 0.4) (layer B.Cu) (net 18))
 (segment (start 147.193 92.075) (end 147.193 95.25) (width 0.4) (layer B.Cu) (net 18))
 (segment (start 147.193 95.25) (end 147.193 96.52) (width 0.4) (layer B.Cu) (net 18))
 (segment (start 142.748 87.63) (end 147.193 92.075) (width 0.4) (layer B.Cu) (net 18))
 (segment (start 137.379002 106.968998) (end 139.573 104.775) (width 0.4) (layer B.Cu) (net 18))
 (segment (start 126.238 109.347) (end 128.616002 106.968998) (width 0.4) (layer B.Cu) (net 18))
 (segment (start 136.652 106.968998) (end 137.379002 106.968998) (width 0.4) (layer B.Cu) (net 18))
 (segment (start 128.616002 106.968998) (end 136.652 106.968998) (width 0.4) (layer B.Cu) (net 18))
 (via (at 139.573 104.775) (size 1.4) (drill 0.6) (layers F.Cu B.Cu) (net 18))
 (segment (start 139.573 104.775) (end 139.573 106.68) (width 0.4) (layer F.Cu) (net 18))
 (segment (start 140.843 107.95) (end 140.843 111.125) (width 0.4) (layer F.Cu) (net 18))
 (segment (start 139.573 106.68) (end 140.843 107.95) (width 0.4) (layer F.Cu) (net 18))
 (segment (start 142.113 112.395) (end 149.733 112.395) (width 0.4) (layer F.Cu) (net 18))
 (segment (start 142.113 112.395) (end 140.843 111.125) (width 0.4) (layer F.Cu) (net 18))
 (via (at 151.638 110.49) (size 1.4) (drill 0.6) (layers F.Cu B.Cu) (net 18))
 (segment (start 151.638 110.49) (end 149.733 112.395) (width 0.4) (layer F.Cu) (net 18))
 (segment (start 153.358996 108.769004) (end 151.638 110.49) (width 0.4) (layer B.Cu) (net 18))
 (segment (start 154.813 108.769004) (end 153.358996 108.769004) (width 0.4) (layer B.Cu) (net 18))
 (segment (start 141.478 87.63) (end 141.478 87.734994) (width 0.4) (layer B.Cu) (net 18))
 (segment (start 133.858 88.369994) (end 135.128 89.639994) (width 0.4) (layer B.Cu) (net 18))
 (segment (start 137.414 78.486) (end 137.414 75.565) (width 0.4) (layer B.Cu) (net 18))
 (segment (start 137.414 78.486) (end 141.478 82.55) (width 0.4) (layer B.Cu) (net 18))
 (segment (start 141.478 82.55) (end 141.478 87.63) (width 0.4) (layer B.Cu) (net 18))
 (segment (start 135.128 89.639994) (end 138.938 89.639994) (width 0.4) (layer B.Cu) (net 18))
 (segment (start 139.573 89.639994) (end 138.938 89.639994) (width 0.4) (layer B.Cu) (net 18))
 (segment (start 141.478 87.734994) (end 139.573 89.639994) (width 0.4) (layer B.Cu) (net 18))
 (segment (start 133.858 88.265) (end 133.858 88.369994) (width 0.4) (layer B.Cu) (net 18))
 (segment (start 157.988 108.769004) (end 159.073996 109.855) (width 0.4) (layer B.Cu) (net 18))
 (segment (start 157.988 108.769004) (end 154.813 108.769004) (width 0.4) (layer B.Cu) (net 18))
 (segment (start 154.813 108.769004) (end 153.543 108.769004) (width 0.4) (layer B.Cu) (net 18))
 (segment (start 159.258 109.855) (end 159.073996 109.855) (width 0.4) (layer B.Cu) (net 18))
 (segment (start 126.238 109.855) (end 126.238 109.347) (width 0.4) (layer B.Cu) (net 18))
 (segment (start 143.383 86.36) (end 144.653 86.36) (width 0.4) (layer F.Cu) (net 13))
 (segment (start 144.653 86.36) (end 145.288 85.725) (width 0.4) (layer F.Cu) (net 13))
 (segment (start 172.466 108.724) (end 172.732 108.724) (width 0.4) (layer B.Cu) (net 13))
 (segment (start 172.732 108.724) (end 173.228 109.22) (width 0.4) (layer B.Cu) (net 13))
 (segment (start 173.228 112.395) (end 173.228 109.22) (width 0.4) (layer B.Cu) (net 13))
 (segment (start 166.509 108.724) (end 172.466 108.724) (width 0.4) (layer B.Cu) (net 13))
 (segment (start 166.509 108.724) (end 165.378 109.855) (width 0.4) (layer B.Cu) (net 13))
 (segment (start 171.958 114.935) (end 171.958 113.665) (width 0.4) (layer B.Cu) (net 13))
 (segment (start 171.958 123.825) (end 171.958 114.935) (width 0.4) (layer B.Cu) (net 13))
 (segment (start 171.958 113.665) (end 173.228 112.395) (width 0.4) (layer B.Cu) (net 13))
 (segment (start 139.573 93.345) (end 139.573 90.17) (width 0.4) (layer F.Cu) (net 13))
 (segment (start 137.668 91.44) (end 139.573 93.345) (width 0.4) (layer B.Cu) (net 13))
 (via (at 139.573 93.345) (size 1.4) (drill 0.6) (layers F.Cu B.Cu) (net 13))
 (segment (start 127.738 88.265) (end 127.738 90.4) (width 0.4) (layer B.Cu) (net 13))
 (segment (start 128.778 91.44) (end 137.668 91.44) (width 0.4) (layer B.Cu) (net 13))
 (segment (start 127.738 90.4) (end 128.778 91.44) (width 0.4) (layer B.Cu) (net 13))
 (segment (start 149.733 85.725) (end 151.638 87.63) (width 0.4) (layer F.Cu) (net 13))
 (segment (start 145.288 85.725) (end 149.733 85.725) (width 0.4) (layer F.Cu) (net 13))
 (segment (start 139.573 90.17) (end 143.383 86.36) (width 0.4) (layer F.Cu) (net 13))
 (segment (start 147.193 104.775) (end 147.193 104.809998) (width 0.4) (layer B.Cu) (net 13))
 (segment (start 147.193 104.809998) (end 149.352 106.968998) (width 0.4) (layer B.Cu) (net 13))
 (segment (start 147.193 104.775) (end 149.098 102.87) (width 0.4) (layer F.Cu) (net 13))
 (segment (start 151.638 93.345) (end 151.638 87.63) (width 0.4) (layer F.Cu) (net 13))
 (segment (start 149.098 95.885) (end 151.638 93.345) (width 0.4) (layer F.Cu) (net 13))
 (segment (start 149.098 102.87) (end 149.098 95.885) (width 0.4) (layer F.Cu) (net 13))
 (segment (start 153.901994 89.893994) (end 151.638 87.63) (width 0.4) (layer B.Cu) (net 13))
 (via (at 151.638 87.63) (size 1.4) (drill 0.6) (layers F.Cu B.Cu) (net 13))
 (segment (start 159.258 89.893994) (end 160.758 88.393994) (width 0.4) (layer B.Cu) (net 13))
 (segment (start 159.258 89.893994) (end 154.178 89.893994) (width 0.4) (layer B.Cu) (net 13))
 (segment (start 154.178 89.893994) (end 153.901994 89.893994) (width 0.4) (layer B.Cu) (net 13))
 (segment (start 160.758 88.265) (end 160.758 88.393994) (width 0.4) (layer B.Cu) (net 13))
 (segment (start 132.358 109.761004) (end 133.35 108.769004) (width 0.4) (layer B.Cu) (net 13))
 (segment (start 133.35 108.769004) (end 136.652 108.769004) (width 0.4) (layer B.Cu) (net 13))
 (segment (start 136.652 108.769004) (end 139.573 108.769004) (width 0.4) (layer B.Cu) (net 13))
 (segment (start 143.198996 108.769004) (end 147.193 104.775) (width 0.4) (layer B.Cu) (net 13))
 (via (at 147.193 104.775) (size 1.4) (drill 0.6) (layers F.Cu B.Cu) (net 13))
 (segment (start 139.573 108.769004) (end 143.198996 108.769004) (width 0.4) (layer B.Cu) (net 13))
 (segment (start 149.352 106.968998) (end 152.908 106.968998) (width 0.4) (layer B.Cu) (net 13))
 (segment (start 132.358 109.855) (end 132.358 109.761004) (width 0.4) (layer B.Cu) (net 13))
 (segment (start 165.378 109.855) (end 165.378 109.371) (width 0.4) (layer B.Cu) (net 13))
 (segment (start 165.378 109.371) (end 162.975998 106.968998) (width 0.4) (layer B.Cu) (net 13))
 (segment (start 162.975998 106.968998) (end 152.908 106.968998) (width 0.4) (layer B.Cu) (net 13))
 (segment (start 152.908 106.968998) (end 152.654 106.968998) (width 0.4) (layer B.Cu) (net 13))
 (segment (start 165.378 109.855) (end 165.378 109.625) (width 0.4) (layer B.Cu) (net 13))
 (segment (start 174.498 123.825) (end 174.498 121.285) (width 0.4) (layer B.Cu) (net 14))
 (segment (start 165.608 107.95) (end 151.638 107.95) (width 0.4) (layer F.Cu) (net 14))
 (segment (start 151.638 107.95) (end 149.098 110.49) (width 0.4) (layer F.Cu) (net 14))
 (segment (start 174.498 121.285) (end 173.228 120.015) (width 0.4) (layer B.Cu) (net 14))
 (via (at 173.228 120.015) (size 1.4) (drill 0.6) (layers F.Cu B.Cu) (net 14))
 (segment (start 173.228 120.015) (end 173.228 109.22) (width 0.4) (layer F.Cu) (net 14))
 (segment (start 173.228 109.22) (end 171.958 107.95) (width 0.4) (layer F.Cu) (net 14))
 (segment (start 171.958 107.95) (end 165.608 107.95) (width 0.4) (layer F.Cu) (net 14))
 (segment (start 146.558 87.63) (end 144.653 87.63) (width 0.4) (layer F.Cu) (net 14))
 (segment (start 142.748 91.44) (end 144.653 93.345) (width 0.4) (layer F.Cu) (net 14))
 (segment (start 142.748 89.535) (end 142.748 91.44) (width 0.4) (layer F.Cu) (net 14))
 (segment (start 144.653 87.63) (end 142.748 89.535) (width 0.4) (layer F.Cu) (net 14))
 (segment (start 138.938 90.239996) (end 141.547996 90.239996) (width 0.4) (layer B.Cu) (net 14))
 (segment (start 131.818 89.469996) (end 132.588 90.239996) (width 0.4) (layer B.Cu) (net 14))
 (segment (start 132.588 90.239996) (end 138.938 90.239996) (width 0.4) (layer B.Cu) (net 14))
 (segment (start 131.818 89.469996) (end 131.818 88.265) (width 0.4) (layer B.Cu) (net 14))
 (via (at 144.653 93.345) (size 1.4) (drill 0.6) (layers F.Cu B.Cu) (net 14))
 (segment (start 141.547996 90.239996) (end 144.653 93.345) (width 0.4) (layer B.Cu) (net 14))
 (segment (start 142.113 108.585) (end 142.113 109.22) (width 0.4) (layer F.Cu) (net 14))
 (segment (start 142.113 109.22) (end 144.653 111.76) (width 0.4) (layer F.Cu) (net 14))
 (segment (start 144.653 111.76) (end 147.828 111.76) (width 0.4) (layer F.Cu) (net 14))
 (segment (start 147.828 111.76) (end 149.098 110.49) (width 0.4) (layer F.Cu) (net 14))
 (segment (start 142.113 104.775) (end 142.113 108.585) (width 0.4) (layer F.Cu) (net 14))
 (segment (start 151.418998 108.169002) (end 149.098 110.49) (width 0.4) (layer B.Cu) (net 14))
 (segment (start 159.858002 108.169002) (end 151.418998 108.169002) (width 0.4) (layer B.Cu) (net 14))
 (segment (start 159.858002 108.169002) (end 161.298 109.609) (width 0.4) (layer B.Cu) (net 14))
 (via (at 149.098 110.49) (size 1.4) (drill 0.6) (layers F.Cu B.Cu) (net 14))
 (segment (start 147.828 94.615) (end 147.828 99.06) (width 0.4) (layer F.Cu) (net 14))
 (segment (start 147.828 99.06) (end 147.193 99.695) (width 0.4) (layer F.Cu) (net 14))
 (segment (start 146.558 87.63) (end 150.368 91.44) (width 0.4) (layer F.Cu) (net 14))
 (segment (start 147.193 99.695) (end 142.113 104.775) (width 0.4) (layer F.Cu) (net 14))
 (segment (start 150.368 92.075) (end 147.828 94.615) (width 0.4) (layer F.Cu) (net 14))
 (segment (start 150.368 91.44) (end 150.368 92.075) (width 0.4) (layer F.Cu) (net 14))
 (segment (start 154.178 91.093998) (end 150.021998 91.093998) (width 0.4) (layer B.Cu) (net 14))
 (segment (start 150.021998 91.093998) (end 146.558 87.63) (width 0.4) (layer B.Cu) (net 14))
 (via (at 146.558 87.63) (size 1.4) (drill 0.6) (layers F.Cu B.Cu) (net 14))
 (segment (start 164.838 88.688998) (end 162.433 91.093998) (width 0.4) (layer B.Cu) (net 14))
 (segment (start 162.433 91.093998) (end 154.178 91.093998) (width 0.4) (layer B.Cu) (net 14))
 (segment (start 164.838 88.265) (end 164.838 88.688998) (width 0.4) (layer B.Cu) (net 14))
 (segment (start 128.278 109.085) (end 129.794 107.569) (width 0.4) (layer B.Cu) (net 14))
 (segment (start 135.763 107.569) (end 139.319 107.569) (width 0.4) (layer B.Cu) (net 14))
 (via (at 142.113 104.775) (size 1.4) (drill 0.6) (layers F.Cu B.Cu) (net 14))
 (segment (start 139.319 107.569) (end 142.113 104.775) (width 0.4) (layer B.Cu) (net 14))
 (segment (start 129.794 107.569) (end 135.763 107.569) (width 0.4) (layer B.Cu) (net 14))
 (segment (start 161.298 109.855) (end 161.298 109.609) (width 0.4) (layer B.Cu) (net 14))
 (segment (start 128.278 109.855) (end 128.278 109.085) (width 0.4) (layer B.Cu) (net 14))
 (segment (start 122.948 105.045) (end 122.948 105.618996) (width 0.4) (layer B.Cu) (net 22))
 (segment (start 134.378 105.045) (end 134.378 104.255) (width 0.4) (layer B.Cu) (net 21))
 (segment (start 127.258 111.635) (end 127.258 112.35853) (width 0.4) (layer B.Cu) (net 37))
 (segment (start 169.418 104.775) (end 169.688 105.045) (width 0.4) (layer B.Cu) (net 46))
 (segment (start 156.448 93.075) (end 156.448 93.615) (width 0.4) (layer B.Cu) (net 48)))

